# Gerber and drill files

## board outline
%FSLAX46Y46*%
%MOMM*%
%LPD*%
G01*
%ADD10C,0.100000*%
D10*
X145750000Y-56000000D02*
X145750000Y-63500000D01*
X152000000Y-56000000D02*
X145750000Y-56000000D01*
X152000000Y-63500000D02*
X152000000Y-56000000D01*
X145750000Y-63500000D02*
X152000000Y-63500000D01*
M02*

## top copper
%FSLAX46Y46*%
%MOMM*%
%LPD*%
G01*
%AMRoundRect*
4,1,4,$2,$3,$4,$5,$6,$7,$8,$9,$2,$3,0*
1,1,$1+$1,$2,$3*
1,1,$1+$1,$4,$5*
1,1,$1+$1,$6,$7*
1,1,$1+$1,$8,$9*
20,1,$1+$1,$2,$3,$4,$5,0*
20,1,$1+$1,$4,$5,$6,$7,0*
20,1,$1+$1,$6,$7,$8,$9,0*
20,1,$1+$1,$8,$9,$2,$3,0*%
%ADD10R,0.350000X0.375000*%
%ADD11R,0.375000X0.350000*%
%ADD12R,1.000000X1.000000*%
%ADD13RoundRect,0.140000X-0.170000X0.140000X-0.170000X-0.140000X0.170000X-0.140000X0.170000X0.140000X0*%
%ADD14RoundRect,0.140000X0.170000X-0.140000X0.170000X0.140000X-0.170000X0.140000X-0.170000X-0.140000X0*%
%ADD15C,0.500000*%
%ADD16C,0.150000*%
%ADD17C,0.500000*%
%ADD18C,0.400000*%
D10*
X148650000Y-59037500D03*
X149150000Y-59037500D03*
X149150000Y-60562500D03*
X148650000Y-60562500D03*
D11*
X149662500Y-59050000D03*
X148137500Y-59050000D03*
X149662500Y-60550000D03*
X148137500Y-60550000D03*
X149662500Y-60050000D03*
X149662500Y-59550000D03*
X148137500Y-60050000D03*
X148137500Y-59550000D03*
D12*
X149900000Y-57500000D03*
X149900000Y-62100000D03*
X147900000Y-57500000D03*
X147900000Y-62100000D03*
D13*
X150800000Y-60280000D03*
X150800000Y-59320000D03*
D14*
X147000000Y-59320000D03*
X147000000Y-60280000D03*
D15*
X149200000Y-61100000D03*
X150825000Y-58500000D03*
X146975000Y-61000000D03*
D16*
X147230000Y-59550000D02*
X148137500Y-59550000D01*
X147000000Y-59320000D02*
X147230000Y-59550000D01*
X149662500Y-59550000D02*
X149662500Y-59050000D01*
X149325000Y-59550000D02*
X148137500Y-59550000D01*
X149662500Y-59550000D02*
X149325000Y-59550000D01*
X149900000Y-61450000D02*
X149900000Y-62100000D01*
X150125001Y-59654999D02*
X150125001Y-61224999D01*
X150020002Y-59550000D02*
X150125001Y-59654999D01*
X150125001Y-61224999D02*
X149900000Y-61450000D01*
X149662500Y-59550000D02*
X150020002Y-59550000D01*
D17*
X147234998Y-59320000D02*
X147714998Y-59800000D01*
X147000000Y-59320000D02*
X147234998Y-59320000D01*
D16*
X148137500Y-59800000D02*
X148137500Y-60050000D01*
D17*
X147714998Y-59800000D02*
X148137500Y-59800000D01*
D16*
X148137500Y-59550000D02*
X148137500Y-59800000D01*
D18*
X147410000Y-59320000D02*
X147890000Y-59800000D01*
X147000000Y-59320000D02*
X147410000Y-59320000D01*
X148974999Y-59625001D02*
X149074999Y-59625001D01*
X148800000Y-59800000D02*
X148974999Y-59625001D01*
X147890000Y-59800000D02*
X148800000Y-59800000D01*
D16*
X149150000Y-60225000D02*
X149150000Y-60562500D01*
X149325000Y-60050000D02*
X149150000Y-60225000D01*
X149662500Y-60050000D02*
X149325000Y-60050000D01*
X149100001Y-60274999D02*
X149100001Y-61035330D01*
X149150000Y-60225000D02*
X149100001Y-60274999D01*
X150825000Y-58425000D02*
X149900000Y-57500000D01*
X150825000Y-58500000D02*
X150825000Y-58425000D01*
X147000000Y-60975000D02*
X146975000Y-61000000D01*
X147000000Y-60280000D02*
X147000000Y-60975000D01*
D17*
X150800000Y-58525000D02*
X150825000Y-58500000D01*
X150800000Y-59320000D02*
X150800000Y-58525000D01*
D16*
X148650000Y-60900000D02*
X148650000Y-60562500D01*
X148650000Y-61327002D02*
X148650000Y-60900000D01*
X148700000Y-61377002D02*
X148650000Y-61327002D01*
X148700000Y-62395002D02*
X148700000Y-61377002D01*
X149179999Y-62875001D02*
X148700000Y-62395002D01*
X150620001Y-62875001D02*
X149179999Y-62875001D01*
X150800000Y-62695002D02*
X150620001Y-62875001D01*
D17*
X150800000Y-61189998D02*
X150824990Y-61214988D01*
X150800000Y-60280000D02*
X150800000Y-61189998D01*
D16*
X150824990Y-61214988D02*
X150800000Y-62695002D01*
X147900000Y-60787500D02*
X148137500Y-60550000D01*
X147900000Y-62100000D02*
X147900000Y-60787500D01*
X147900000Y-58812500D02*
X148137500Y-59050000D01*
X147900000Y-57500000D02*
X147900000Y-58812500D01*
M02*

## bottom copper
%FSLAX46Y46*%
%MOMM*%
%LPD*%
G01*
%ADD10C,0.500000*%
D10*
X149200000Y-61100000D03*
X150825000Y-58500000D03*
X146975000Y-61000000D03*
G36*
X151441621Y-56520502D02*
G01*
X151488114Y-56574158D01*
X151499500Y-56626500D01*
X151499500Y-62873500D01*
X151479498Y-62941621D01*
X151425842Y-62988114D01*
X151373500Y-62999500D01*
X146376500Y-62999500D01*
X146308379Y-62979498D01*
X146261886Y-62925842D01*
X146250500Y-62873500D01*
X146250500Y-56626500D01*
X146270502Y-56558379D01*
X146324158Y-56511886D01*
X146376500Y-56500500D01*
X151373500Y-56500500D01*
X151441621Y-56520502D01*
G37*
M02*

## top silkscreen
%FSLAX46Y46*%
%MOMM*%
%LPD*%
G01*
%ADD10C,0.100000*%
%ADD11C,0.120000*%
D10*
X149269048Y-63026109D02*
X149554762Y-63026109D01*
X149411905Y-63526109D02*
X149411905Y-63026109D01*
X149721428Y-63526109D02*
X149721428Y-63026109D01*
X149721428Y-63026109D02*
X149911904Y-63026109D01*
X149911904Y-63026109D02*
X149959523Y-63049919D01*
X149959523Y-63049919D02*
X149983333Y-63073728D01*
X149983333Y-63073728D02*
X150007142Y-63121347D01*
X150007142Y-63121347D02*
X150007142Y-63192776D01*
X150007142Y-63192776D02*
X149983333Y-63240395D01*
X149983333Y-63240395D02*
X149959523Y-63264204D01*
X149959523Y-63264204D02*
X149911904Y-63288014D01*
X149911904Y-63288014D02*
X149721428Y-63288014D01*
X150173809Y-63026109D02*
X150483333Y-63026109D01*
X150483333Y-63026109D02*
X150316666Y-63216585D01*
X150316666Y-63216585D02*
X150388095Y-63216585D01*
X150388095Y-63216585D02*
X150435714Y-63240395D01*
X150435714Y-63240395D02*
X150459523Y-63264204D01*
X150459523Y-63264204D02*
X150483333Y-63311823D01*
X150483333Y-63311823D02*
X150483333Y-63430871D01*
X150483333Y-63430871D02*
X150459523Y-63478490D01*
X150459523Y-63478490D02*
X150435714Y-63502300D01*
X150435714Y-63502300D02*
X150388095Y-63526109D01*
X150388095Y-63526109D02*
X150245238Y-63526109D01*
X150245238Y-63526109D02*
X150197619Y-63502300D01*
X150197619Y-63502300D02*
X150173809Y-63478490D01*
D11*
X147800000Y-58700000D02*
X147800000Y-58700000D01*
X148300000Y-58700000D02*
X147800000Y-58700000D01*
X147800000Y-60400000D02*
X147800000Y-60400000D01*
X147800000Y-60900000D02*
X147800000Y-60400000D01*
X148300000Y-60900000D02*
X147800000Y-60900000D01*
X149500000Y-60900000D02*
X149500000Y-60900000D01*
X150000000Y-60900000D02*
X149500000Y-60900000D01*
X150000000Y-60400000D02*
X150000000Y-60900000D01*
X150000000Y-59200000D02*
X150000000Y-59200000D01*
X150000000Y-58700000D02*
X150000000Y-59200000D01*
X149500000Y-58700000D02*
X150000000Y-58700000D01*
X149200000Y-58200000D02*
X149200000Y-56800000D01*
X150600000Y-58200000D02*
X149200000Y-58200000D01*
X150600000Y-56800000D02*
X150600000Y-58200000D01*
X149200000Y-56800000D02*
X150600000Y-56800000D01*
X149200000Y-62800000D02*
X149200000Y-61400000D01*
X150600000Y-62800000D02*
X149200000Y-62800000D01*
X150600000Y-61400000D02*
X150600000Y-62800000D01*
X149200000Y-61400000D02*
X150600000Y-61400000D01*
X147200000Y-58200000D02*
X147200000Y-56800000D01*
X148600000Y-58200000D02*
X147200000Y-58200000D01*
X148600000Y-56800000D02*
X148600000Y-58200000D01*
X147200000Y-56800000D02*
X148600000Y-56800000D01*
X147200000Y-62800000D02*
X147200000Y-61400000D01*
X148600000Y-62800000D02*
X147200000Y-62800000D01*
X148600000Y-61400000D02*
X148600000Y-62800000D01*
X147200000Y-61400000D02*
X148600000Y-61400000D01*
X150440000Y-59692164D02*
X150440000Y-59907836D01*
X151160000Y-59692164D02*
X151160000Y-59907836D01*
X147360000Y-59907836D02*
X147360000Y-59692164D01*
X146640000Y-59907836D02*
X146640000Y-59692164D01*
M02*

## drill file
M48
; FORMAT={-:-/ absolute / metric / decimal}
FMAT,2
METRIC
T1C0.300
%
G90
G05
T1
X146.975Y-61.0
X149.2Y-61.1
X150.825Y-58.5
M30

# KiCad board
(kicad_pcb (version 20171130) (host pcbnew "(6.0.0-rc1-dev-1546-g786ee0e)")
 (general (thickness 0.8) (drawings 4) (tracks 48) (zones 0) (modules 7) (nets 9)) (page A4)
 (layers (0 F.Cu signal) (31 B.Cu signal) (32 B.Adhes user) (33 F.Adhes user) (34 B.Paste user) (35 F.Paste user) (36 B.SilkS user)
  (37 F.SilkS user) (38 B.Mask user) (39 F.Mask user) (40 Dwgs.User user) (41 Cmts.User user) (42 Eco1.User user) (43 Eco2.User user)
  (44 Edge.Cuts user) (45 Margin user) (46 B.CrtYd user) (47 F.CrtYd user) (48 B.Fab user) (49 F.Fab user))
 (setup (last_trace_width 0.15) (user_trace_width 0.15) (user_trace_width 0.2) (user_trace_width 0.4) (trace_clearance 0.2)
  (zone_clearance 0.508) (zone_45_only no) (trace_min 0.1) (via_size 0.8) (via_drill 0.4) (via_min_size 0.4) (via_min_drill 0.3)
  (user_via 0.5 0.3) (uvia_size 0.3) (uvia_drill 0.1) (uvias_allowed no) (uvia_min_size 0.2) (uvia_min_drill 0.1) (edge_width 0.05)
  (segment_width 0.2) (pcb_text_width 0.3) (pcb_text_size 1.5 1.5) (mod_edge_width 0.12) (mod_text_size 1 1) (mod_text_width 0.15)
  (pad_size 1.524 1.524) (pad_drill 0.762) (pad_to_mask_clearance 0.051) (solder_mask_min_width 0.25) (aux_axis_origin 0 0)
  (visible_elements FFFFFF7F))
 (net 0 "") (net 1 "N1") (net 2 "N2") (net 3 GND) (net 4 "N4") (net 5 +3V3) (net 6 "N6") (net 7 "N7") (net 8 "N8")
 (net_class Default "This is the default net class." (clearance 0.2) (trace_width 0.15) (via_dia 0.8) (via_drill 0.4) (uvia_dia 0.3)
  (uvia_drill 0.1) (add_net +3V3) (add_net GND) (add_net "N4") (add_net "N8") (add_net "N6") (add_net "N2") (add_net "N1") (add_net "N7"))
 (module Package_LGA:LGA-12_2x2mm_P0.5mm (layer F.Cu) (at 148.9 59.8)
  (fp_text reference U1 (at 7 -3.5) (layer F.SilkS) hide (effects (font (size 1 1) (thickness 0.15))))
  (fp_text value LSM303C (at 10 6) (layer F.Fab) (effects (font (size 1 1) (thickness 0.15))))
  (fp_line (start -1.1 -1.1) (end -1.1 -1.1) (layer F.SilkS) (width 0.12))
  (fp_line (start -0.6 -1.1) (end -1.1 -1.1) (layer F.SilkS) (width 0.12))
  (fp_line (start -1.1 0.6) (end -1.1 0.6) (layer F.SilkS) (width 0.12))
  (fp_line (start -1.1 1.1) (end -1.1 0.6) (layer F.SilkS) (width 0.12))
  (fp_line (start -0.6 1.1) (end -1.1 1.1) (layer F.SilkS) (width 0.12))
  (fp_line (start 0.6 1.1) (end 0.6 1.1) (layer F.SilkS) (width 0.12))
  (fp_line (start 1.1 1.1) (end 0.6 1.1) (layer F.SilkS) (width 0.12))
  (fp_line (start 1.1 0.6) (end 1.1 1.1) (layer F.SilkS) (width 0.12))
  (fp_line (start 1.1 -0.6) (end 1.1 -0.6) (layer F.SilkS) (width 0.12))
  (fp_line (start 1.1 -1.1) (end 1.1 -0.6) (layer F.SilkS) (width 0.12))
  (fp_line (start 0.6 -1.1) (end 1.1 -1.1) (layer F.SilkS) (width 0.12))
  (pad 12 smd rect (at -0.25 -0.7625 90) (size 0.375 0.35) (layers F.Cu F.Paste F.Mask) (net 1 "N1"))
  (pad 11 smd rect (at 0.25 -0.7625 90) (size 0.375 0.35) (layers F.Cu F.Paste F.Mask) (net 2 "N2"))
  (pad 6 smd rect (at 0.25 0.7625 90) (size 0.375 0.35) (layers F.Cu F.Paste F.Mask) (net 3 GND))
  (pad 5 smd rect (at -0.25 0.7625 90) (size 0.375 0.35) (layers F.Cu F.Paste F.Mask) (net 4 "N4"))
  (pad 10 smd rect (at 0.7625 -0.75) (size 0.375 0.35) (layers F.Cu F.Paste F.Mask) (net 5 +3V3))
  (pad 1 smd rect (at -0.7625 -0.75) (size 0.375 0.35) (layers F.Cu F.Paste F.Mask) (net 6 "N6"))
  (pad 7 smd rect (at 0.7625 0.75) (size 0.375 0.35) (layers F.Cu F.Paste F.Mask) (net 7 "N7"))
  (pad 4 smd rect (at -0.7625 0.75) (size 0.375 0.35) (layers F.Cu F.Paste F.Mask) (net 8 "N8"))
  (pad 8 smd rect (at 0.7625 0.25) (size 0.375 0.35) (layers F.Cu F.Paste F.Mask) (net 3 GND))
  (pad 9 smd rect (at 0.7625 -0.25) (size 0.375 0.35) (layers F.Cu F.Paste F.Mask) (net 5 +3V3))
  (pad 3 smd rect (at -0.7625 0.25) (size 0.375 0.35) (layers F.Cu F.Paste F.Mask) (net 5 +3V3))
  (pad 2 smd rect (at -0.7625 -0.25) (size 0.375 0.35) (layers F.Cu F.Paste F.Mask) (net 5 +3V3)))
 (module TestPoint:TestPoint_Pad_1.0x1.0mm (layer F.Cu) (at 149.9 57.5)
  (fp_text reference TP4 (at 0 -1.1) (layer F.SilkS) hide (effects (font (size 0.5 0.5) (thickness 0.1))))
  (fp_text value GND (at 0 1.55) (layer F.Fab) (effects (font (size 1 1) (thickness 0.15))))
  (fp_line (start -0.7 0.7) (end -0.7 -0.7) (layer F.SilkS) (width 0.12))
  (fp_line (start 0.7 0.7) (end -0.7 0.7) (layer F.SilkS) (width 0.12))
  (fp_line (start 0.7 -0.7) (end 0.7 0.7) (layer F.SilkS) (width 0.12))
  (fp_line (start -0.7 -0.7) (end 0.7 -0.7) (layer F.SilkS) (width 0.12))
  (pad 1 smd rect (at 0 0) (size 1 1) (layers F.Cu F.Mask) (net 3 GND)))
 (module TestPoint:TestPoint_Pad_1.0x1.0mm (layer F.Cu) (at 149.9 62.1)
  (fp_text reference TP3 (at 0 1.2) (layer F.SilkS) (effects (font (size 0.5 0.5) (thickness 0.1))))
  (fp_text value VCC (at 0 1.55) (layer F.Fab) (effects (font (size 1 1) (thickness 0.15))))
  (fp_line (start -0.7 0.7) (end -0.7 -0.7) (layer F.SilkS) (width 0.12))
  (fp_line (start 0.7 0.7) (end -0.7 0.7) (layer F.SilkS) (width 0.12))
  (fp_line (start 0.7 -0.7) (end 0.7 0.7) (layer F.SilkS) (width 0.12))
  (fp_line (start -0.7 -0.7) (end 0.7 -0.7) (layer F.SilkS) (width 0.12))
  (pad 1 smd rect (at 0 0) (size 1 1) (layers F.Cu F.Mask) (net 5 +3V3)))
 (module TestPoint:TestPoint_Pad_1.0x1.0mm (layer F.Cu) (at 147.9 57.5)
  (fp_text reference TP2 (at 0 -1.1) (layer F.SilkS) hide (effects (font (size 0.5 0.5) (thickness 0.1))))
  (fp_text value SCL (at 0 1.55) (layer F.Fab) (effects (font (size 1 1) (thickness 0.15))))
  (fp_line (start -0.7 0.7) (end -0.7 -0.7) (layer F.SilkS) (width 0.12))
  (fp_line (start 0.7 0.7) (end -0.7 0.7) (layer F.SilkS) (width 0.12))
  (fp_line (start 0.7 -0.7) (end 0.7 0.7) (layer F.SilkS) (width 0.12))
  (fp_line (start -0.7 -0.7) (end 0.7 -0.7) (layer F.SilkS) (width 0.12))
  (pad 1 smd rect (at 0 0) (size 1 1) (layers F.Cu F.Mask) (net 6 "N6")))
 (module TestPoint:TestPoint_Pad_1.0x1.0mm (layer F.Cu) (at 147.9 62.1)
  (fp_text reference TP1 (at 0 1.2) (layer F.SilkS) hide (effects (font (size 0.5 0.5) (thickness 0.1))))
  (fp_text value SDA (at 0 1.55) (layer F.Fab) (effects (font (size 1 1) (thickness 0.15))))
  (fp_line (start -0.7 0.7) (end -0.7 -0.7) (layer F.SilkS) (width 0.12))
  (fp_line (start 0.7 0.7) (end -0.7 0.7) (layer F.SilkS) (width 0.12))
  (fp_line (start 0.7 -0.7) (end 0.7 0.7) (layer F.SilkS) (width 0.12))
  (fp_line (start -0.7 -0.7) (end 0.7 -0.7) (layer F.SilkS) (width 0.12))
  (pad 1 smd rect (at 0 0) (size 1 1) (layers F.Cu F.Mask) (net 8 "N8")))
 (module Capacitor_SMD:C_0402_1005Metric (layer F.Cu) (at 150.8 59.8 270)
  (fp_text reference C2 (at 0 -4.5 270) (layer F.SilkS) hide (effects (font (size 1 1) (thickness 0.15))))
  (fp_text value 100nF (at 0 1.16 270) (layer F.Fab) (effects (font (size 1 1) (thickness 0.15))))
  (fp_line (start -0.107836 0.36) (end 0.107836 0.36) (layer F.SilkS) (width 0.12))
  (fp_line (start -0.107836 -0.36) (end 0.107836 -0.36) (layer F.SilkS) (width 0.12))
  (pad 2 smd roundrect (at 0.48 0 270) (size 0.56 0.62) (layers F.Cu F.Paste F.Mask) (roundrect_rratio 0.25) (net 4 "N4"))
  (pad 1 smd roundrect (at -0.48 0 270) (size 0.56 0.62) (layers F.Cu F.Paste F.Mask) (roundrect_rratio 0.25) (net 3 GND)))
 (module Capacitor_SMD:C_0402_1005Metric (layer F.Cu) (at 147 59.8 90)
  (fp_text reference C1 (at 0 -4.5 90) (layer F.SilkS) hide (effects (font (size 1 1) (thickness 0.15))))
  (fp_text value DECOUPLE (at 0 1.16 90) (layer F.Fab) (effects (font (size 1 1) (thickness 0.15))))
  (fp_line (start -0.107836 0.36) (end 0.107836 0.36) (layer F.SilkS) (width 0.12))
  (fp_line (start -0.107836 -0.36) (end 0.107836 -0.36) (layer F.SilkS) (width 0.12))
  (pad 2 smd roundrect (at 0.48 0 90) (size 0.56 0.62) (layers F.Cu F.Paste F.Mask) (roundrect_rratio 0.25) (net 5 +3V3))
  (pad 1 smd roundrect (at -0.48 0 90) (size 0.56 0.62) (layers F.Cu F.Paste F.Mask) (roundrect_rratio 0.25) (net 3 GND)))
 (gr_line (start 145.75 56) (end 145.75 63.5) (layer Edge.Cuts) (width 0.1))
 (gr_line (start 152 56) (end 145.75 56) (layer Edge.Cuts) (width 0.1))
 (gr_line (start 152 63.5) (end 152 56) (layer Edge.Cuts) (width 0.1))
 (gr_line (start 145.75 63.5) (end 152 63.5) (layer Edge.Cuts) (width 0.1))
 (segment (start 147.23 59.55) (end 148.1375 59.55) (width 0.15) (layer F.Cu) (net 5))
 (segment (start 147 59.32) (end 147.23 59.55) (width 0.15) (layer F.Cu) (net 5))
 (segment (start 149.6625 59.55) (end 149.6625 59.05) (width 0.15) (layer F.Cu) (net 5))
 (segment (start 149.325 59.55) (end 148.1375 59.55) (width 0.15) (layer F.Cu) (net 5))
 (segment (start 149.6625 59.55) (end 149.325 59.55) (width 0.15) (layer F.Cu) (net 5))
 (segment (start 149.9 61.45) (end 149.9 62.1) (width 0.15) (layer F.Cu) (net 5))
 (segment (start 150.125001 59.654999) (end 150.125001 61.224999) (width 0.15) (layer F.Cu) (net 5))
 (segment (start 150.020002 59.55) (end 150.125001 59.654999) (width 0.15) (layer F.Cu) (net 5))
 (segment (start 150.125001 61.224999) (end 149.9 61.45) (width 0.15) (layer F.Cu) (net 5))
 (segment (start 149.6625 59.55) (end 150.020002 59.55) (width 0.15) (layer F.Cu) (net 5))
 (segment (start 147.234998 59.32) (end 147.714998 59.8) (width 0.5) (layer F.Cu) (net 5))
 (segment (start 147 59.32) (end 147.234998 59.32) (width 0.5) (layer F.Cu) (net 5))
 (segment (start 148.1375 59.8) (end 148.1375 60.05) (width 0.15) (layer F.Cu) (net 5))
 (segment (start 147.714998 59.8) (end 148.1375 59.8) (width 0.5) (layer F.Cu) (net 5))
 (segment (start 148.1375 59.55) (end 148.1375 59.8) (width 0.15) (layer F.Cu) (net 5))
 (segment (start 147.41 59.32) (end 147.89 59.8) (width 0.4) (layer F.Cu) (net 5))
 (segment (start 147 59.32) (end 147.41 59.32) (width 0.4) (layer F.Cu) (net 5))
 (segment (start 148.974999 59.625001) (end 149.074999 59.625001) (width 0.4) (layer F.Cu) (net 5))
 (segment (start 148.8 59.8) (end 148.974999 59.625001) (width 0.4) (layer F.Cu) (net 5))
 (segment (start 147.89 59.8) (end 148.8 59.8) (width 0.4) (layer F.Cu) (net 5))
 (segment (start 149.15 60.225) (end 149.15 60.5625) (width 0.15) (layer F.Cu) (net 3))
 (segment (start 149.325 60.05) (end 149.15 60.225) (width 0.15) (layer F.Cu) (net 3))
 (segment (start 149.6625 60.05) (end 149.325 60.05) (width 0.15) (layer F.Cu) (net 3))
 (via (at 149.2 61.1) (size 0.5) (drill 0.3) (layers F.Cu B.Cu) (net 3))
 (segment (start 149.100001 60.274999) (end 149.100001 61.03533) (width 0.15) (layer F.Cu) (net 3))
 (segment (start 149.15 60.225) (end 149.100001 60.274999) (width 0.15) (layer F.Cu) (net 3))
 (via (at 150.825 58.5) (size 0.5) (drill 0.3) (layers F.Cu B.Cu) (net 3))
 (segment (start 150.825 58.425) (end 149.9 57.5) (width 0.15) (layer F.Cu) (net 3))
 (segment (start 150.825 58.5) (end 150.825 58.425) (width 0.15) (layer F.Cu) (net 3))
 (via (at 146.975 61) (size 0.5) (drill 0.3) (layers F.Cu B.Cu) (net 3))
 (segment (start 147 60.975) (end 146.975 61) (width 0.15) (layer F.Cu) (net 3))
 (segment (start 147 60.28) (end 147 60.975) (width 0.15) (layer F.Cu) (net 3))
 (segment (start 150.8 58.525) (end 150.825 58.5) (width 0.5) (layer F.Cu) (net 3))
 (segment (start 150.8 59.32) (end 150.8 58.525) (width 0.5) (layer F.Cu) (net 3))
 (segment (start 148.65 60.9) (end 148.65 60.5625) (width 0.15) (layer F.Cu) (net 4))
 (segment (start 148.65 61.327002) (end 148.65 60.9) (width 0.15) (layer F.Cu) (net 4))
 (segment (start 148.7 61.377002) (end 148.65 61.327002) (width 0.15) (layer F.Cu) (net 4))
 (segment (start 148.7 62.395002) (end 148.7 61.377002) (width 0.15) (layer F.Cu) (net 4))
 (segment (start 149.179999 62.875001) (end 148.7 62.395002) (width 0.15) (layer F.Cu) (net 4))
 (segment (start 150.620001 62.875001) (end 149.179999 62.875001) (width 0.15) (layer F.Cu) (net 4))
 (segment (start 150.8 62.695002) (end 150.620001 62.875001) (width 0.15) (layer F.Cu) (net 4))
 (segment (start 150.8 61.189998) (end 150.82499 61.214988) (width 0.5) (layer F.Cu) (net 4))
 (segment (start 150.8 60.28) (end 150.8 61.189998) (width 0.5) (layer F.Cu) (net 4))
 (segment (start 150.82499 61.214988) (end 150.8 62.695002) (width 0.15) (layer F.Cu) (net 4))
 (segment (start 147.9 60.7875) (end 148.1375 60.55) (width 0.15) (layer F.Cu) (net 8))
 (segment (start 147.9 62.1) (end 147.9 60.7875) (width 0.15) (layer F.Cu) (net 8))
 (segment (start 147.9 58.8125) (end 148.1375 59.05) (width 0.15) (layer F.Cu) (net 6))
 (segment (start 147.9 57.5) (end 147.9 58.8125) (width 0.15) (layer F.Cu) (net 6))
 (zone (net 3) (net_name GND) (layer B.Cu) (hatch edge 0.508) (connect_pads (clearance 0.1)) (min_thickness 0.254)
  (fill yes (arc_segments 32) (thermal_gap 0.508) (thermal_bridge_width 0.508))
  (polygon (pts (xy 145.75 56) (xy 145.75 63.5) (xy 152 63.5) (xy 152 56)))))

